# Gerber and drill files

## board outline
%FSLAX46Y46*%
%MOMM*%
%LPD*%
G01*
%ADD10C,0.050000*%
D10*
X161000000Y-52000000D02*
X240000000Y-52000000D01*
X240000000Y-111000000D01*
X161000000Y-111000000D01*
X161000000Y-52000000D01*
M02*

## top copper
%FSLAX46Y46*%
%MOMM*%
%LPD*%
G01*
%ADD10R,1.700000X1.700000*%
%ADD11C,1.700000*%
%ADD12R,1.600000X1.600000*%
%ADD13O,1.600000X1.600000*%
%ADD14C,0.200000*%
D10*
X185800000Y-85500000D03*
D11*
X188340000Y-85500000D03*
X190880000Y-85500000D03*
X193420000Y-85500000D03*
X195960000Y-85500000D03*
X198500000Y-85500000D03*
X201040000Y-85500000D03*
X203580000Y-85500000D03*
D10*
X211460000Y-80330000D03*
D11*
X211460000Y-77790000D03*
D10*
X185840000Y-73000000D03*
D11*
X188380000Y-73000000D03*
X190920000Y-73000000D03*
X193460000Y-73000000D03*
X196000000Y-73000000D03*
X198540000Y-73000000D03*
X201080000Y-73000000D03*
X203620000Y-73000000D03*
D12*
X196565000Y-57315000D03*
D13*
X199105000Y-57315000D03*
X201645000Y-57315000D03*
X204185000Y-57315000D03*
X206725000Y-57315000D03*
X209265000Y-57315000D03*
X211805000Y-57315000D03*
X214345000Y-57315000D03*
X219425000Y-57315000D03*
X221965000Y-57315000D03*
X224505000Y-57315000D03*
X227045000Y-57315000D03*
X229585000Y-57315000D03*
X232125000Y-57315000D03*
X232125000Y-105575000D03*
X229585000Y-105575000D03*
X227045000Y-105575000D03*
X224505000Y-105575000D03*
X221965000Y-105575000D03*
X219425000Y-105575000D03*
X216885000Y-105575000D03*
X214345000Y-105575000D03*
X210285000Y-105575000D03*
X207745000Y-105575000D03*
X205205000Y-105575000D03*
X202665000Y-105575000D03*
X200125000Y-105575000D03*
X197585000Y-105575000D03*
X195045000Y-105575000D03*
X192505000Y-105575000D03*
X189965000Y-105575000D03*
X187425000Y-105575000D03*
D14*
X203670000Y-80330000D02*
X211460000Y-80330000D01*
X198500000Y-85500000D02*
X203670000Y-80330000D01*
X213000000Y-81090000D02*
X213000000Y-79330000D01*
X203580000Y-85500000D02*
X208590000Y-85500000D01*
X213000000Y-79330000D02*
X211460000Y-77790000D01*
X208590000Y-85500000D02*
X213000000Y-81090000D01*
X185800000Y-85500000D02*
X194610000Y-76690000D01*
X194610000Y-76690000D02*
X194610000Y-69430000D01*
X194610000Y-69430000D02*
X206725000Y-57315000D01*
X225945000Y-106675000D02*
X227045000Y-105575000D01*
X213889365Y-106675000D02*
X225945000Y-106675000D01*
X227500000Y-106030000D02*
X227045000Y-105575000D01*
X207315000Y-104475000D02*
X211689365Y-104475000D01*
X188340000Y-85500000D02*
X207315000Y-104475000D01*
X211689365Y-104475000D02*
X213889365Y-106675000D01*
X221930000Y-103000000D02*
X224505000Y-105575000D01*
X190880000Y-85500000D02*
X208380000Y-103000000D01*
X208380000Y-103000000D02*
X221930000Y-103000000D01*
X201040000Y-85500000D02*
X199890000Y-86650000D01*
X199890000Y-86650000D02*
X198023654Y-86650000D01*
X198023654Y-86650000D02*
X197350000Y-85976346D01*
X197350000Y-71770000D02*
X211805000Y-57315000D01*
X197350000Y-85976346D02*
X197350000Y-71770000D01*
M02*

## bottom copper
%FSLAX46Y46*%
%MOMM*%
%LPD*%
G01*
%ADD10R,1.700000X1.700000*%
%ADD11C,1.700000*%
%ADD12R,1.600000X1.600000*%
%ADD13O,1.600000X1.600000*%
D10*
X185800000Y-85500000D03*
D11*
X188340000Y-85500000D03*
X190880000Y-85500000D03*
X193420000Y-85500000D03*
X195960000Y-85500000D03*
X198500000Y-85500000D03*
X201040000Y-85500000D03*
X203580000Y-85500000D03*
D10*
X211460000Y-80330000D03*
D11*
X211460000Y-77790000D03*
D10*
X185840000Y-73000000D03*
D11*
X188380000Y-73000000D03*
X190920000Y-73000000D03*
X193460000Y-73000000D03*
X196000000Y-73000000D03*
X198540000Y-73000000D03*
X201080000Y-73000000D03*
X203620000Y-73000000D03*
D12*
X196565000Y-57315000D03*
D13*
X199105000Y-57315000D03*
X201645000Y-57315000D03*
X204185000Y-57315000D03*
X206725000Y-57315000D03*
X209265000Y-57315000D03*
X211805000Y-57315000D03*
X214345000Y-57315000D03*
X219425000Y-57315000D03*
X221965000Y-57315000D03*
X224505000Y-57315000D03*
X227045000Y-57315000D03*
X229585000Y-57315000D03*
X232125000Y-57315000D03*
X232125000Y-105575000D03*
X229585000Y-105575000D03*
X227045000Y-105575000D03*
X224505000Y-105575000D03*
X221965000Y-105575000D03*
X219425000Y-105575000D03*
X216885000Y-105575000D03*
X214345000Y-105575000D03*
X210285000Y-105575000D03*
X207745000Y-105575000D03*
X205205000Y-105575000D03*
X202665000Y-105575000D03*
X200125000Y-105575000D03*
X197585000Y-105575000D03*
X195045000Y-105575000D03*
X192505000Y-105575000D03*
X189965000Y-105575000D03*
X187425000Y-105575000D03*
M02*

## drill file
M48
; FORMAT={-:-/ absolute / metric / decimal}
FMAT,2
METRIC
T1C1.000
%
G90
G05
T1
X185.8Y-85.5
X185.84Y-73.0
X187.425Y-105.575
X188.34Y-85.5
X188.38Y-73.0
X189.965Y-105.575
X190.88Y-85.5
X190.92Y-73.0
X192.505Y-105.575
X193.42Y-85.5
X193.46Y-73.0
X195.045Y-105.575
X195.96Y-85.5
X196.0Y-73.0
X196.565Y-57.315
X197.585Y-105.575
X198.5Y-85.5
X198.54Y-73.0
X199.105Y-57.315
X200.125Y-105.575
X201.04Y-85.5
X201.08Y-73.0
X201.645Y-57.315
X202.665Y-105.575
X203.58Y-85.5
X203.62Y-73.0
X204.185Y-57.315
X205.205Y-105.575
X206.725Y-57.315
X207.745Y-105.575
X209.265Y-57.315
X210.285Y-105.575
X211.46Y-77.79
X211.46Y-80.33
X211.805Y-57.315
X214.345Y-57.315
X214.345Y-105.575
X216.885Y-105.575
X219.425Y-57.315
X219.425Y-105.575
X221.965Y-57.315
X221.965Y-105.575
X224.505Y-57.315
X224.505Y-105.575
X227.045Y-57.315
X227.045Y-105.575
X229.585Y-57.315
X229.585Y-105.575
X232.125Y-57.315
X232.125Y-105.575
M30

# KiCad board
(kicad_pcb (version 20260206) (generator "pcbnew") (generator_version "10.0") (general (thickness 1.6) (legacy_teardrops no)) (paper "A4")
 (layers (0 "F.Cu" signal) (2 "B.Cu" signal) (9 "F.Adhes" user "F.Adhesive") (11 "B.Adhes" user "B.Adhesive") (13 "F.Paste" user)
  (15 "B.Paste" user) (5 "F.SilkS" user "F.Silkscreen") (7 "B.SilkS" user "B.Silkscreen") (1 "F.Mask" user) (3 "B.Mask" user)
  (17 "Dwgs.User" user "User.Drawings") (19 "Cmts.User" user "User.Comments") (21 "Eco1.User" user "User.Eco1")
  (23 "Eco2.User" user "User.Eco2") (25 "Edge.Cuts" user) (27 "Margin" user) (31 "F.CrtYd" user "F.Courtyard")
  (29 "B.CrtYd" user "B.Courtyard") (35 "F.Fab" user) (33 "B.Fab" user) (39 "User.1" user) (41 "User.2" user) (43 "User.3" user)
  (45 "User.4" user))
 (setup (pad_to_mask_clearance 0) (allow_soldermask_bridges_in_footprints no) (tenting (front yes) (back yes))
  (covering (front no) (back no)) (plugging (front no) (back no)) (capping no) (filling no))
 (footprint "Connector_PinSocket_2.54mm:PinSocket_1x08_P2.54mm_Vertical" (layer "F.Cu") (at 185.8 85.5 90)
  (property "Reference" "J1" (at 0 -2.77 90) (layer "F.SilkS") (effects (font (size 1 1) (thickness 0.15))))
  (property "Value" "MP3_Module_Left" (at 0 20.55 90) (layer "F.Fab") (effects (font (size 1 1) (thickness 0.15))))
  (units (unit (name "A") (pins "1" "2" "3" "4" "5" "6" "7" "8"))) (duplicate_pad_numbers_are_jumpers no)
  (pad "1" thru_hole rect (at 0 0 90) (size 1.7 1.7) (drill 1) (layers "*.Cu" "*.Mask") (remove_unused_layers no) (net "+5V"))
  (pad "2" thru_hole circle (at 0 2.54 90) (size 1.7 1.7) (drill 1) (layers "*.Cu" "*.Mask") (remove_unused_layers no) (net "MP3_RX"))
  (pad "3" thru_hole circle (at 0 5.08 90) (size 1.7 1.7) (drill 1) (layers "*.Cu" "*.Mask") (remove_unused_layers no) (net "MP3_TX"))
  (pad "4" thru_hole circle (at 0 7.62 90) (size 1.7 1.7) (drill 1) (layers "*.Cu" "*.Mask") (remove_unused_layers no)
   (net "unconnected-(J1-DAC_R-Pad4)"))
  (pad "5" thru_hole circle (at 0 10.16 90) (size 1.7 1.7) (drill 1) (layers "*.Cu" "*.Mask") (remove_unused_layers no)
   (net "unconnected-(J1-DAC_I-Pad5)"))
  (pad "6" thru_hole circle (at 0 12.7 90) (size 1.7 1.7) (drill 1) (layers "*.Cu" "*.Mask") (remove_unused_layers no) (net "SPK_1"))
  (pad "7" thru_hole circle (at 0 15.24 90) (size 1.7 1.7) (drill 1) (layers "*.Cu" "*.Mask") (remove_unused_layers no) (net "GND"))
  (pad "8" thru_hole circle (at 0 17.78 90) (size 1.7 1.7) (drill 1) (layers "*.Cu" "*.Mask") (remove_unused_layers no) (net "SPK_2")))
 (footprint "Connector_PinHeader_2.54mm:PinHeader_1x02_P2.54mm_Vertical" (layer "F.Cu") (at 211.46 80.33 180)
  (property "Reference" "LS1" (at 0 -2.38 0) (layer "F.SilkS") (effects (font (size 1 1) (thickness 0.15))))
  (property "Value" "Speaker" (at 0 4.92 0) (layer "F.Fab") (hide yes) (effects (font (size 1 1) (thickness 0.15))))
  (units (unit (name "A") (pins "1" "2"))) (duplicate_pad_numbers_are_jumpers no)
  (pad "1" thru_hole rect (at 0 0 180) (size 1.7 1.7) (drill 1) (layers "*.Cu" "*.Mask") (remove_unused_layers no) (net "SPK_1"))
  (pad "2" thru_hole circle (at 0 2.54 180) (size 1.7 1.7) (drill 1) (layers "*.Cu" "*.Mask") (remove_unused_layers no) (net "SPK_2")))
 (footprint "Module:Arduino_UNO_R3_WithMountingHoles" (layer "F.Cu") (at 115.75 120.70425)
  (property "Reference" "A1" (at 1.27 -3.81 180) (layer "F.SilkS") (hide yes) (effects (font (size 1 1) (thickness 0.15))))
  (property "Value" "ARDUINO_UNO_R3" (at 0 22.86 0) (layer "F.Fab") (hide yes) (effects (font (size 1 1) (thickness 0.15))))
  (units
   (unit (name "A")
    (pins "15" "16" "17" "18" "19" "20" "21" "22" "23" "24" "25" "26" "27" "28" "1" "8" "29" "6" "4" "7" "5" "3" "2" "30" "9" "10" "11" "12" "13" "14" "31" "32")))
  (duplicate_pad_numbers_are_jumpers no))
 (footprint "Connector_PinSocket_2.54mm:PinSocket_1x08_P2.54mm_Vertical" (layer "F.Cu") (at 185.84 73 90)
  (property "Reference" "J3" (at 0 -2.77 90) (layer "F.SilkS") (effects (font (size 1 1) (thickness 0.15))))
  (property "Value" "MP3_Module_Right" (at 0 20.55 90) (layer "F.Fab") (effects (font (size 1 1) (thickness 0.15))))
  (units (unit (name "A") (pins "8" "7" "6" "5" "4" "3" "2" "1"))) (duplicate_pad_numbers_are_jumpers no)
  (pad "1" thru_hole rect (at 0 0 90) (size 1.7 1.7) (drill 1) (layers "*.Cu" "*.Mask") (remove_unused_layers no)
   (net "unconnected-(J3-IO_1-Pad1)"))
  (pad "2" thru_hole circle (at 0 2.54 90) (size 1.7 1.7) (drill 1) (layers "*.Cu" "*.Mask") (remove_unused_layers no)
   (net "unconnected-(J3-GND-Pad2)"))
  (pad "3" thru_hole circle (at 0 5.08 90) (size 1.7 1.7) (drill 1) (layers "*.Cu" "*.Mask") (remove_unused_layers no)
   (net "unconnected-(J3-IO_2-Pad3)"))
  (pad "4" thru_hole circle (at 0 7.62 90) (size 1.7 1.7) (drill 1) (layers "*.Cu" "*.Mask") (remove_unused_layers no)
   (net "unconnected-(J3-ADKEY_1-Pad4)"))
  (pad "5" thru_hole circle (at 0 10.16 90) (size 1.7 1.7) (drill 1) (layers "*.Cu" "*.Mask") (remove_unused_layers no)
   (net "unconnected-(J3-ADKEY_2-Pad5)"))
  (pad "6" thru_hole circle (at 0 12.7 90) (size 1.7 1.7) (drill 1) (layers "*.Cu" "*.Mask") (remove_unused_layers no)
   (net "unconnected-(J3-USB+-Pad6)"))
  (pad "7" thru_hole circle (at 0 15.24 90) (size 1.7 1.7) (drill 1) (layers "*.Cu" "*.Mask") (remove_unused_layers no)
   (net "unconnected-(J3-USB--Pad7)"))
  (pad "8" thru_hole circle (at 0 17.78 90) (size 1.7 1.7) (drill 1) (layers "*.Cu" "*.Mask") (remove_unused_layers no)
   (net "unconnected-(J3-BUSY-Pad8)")))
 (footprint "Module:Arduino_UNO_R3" (layer "F.Cu") (at 196.565 57.315)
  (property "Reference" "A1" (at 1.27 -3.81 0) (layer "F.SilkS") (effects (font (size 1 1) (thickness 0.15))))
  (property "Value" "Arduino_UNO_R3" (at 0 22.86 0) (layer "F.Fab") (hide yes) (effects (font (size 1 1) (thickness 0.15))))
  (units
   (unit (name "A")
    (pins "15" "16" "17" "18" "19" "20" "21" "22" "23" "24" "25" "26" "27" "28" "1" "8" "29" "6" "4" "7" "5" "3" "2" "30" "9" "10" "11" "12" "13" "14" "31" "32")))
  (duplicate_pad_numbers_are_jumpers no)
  (pad "1" thru_hole rect (at 0 0 90) (size 1.6 1.6) (drill 1) (layers "*.Cu" "*.Mask") (remove_unused_layers no)
   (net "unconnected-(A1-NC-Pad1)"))
  (pad "2" thru_hole oval (at 2.54 0 90) (size 1.6 1.6) (drill 1) (layers "*.Cu" "*.Mask") (remove_unused_layers no)
   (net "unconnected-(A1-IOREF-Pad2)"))
  (pad "3" thru_hole oval (at 5.08 0 90) (size 1.6 1.6) (drill 1) (layers "*.Cu" "*.Mask") (remove_unused_layers no)
   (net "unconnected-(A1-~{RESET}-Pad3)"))
  (pad "4" thru_hole oval (at 7.62 0 90) (size 1.6 1.6) (drill 1) (layers "*.Cu" "*.Mask") (remove_unused_layers no)
   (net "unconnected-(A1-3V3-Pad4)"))
  (pad "5" thru_hole oval (at 10.16 0 90) (size 1.6 1.6) (drill 1) (layers "*.Cu" "*.Mask") (remove_unused_layers no) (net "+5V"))
  (pad "6" thru_hole oval (at 12.7 0 90) (size 1.6 1.6) (drill 1) (layers "*.Cu" "*.Mask") (remove_unused_layers no)
   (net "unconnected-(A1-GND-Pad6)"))
  (pad "7" thru_hole oval (at 15.24 0 90) (size 1.6 1.6) (drill 1) (layers "*.Cu" "*.Mask") (remove_unused_layers no) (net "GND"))
  (pad "8" thru_hole oval (at 17.78 0 90) (size 1.6 1.6) (drill 1) (layers "*.Cu" "*.Mask") (remove_unused_layers no)
   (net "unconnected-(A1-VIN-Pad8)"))
  (pad "9" thru_hole oval (at 22.86 0 90) (size 1.6 1.6) (drill 1) (layers "*.Cu" "*.Mask") (remove_unused_layers no)
   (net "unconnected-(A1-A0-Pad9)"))
  (pad "10" thru_hole oval (at 25.4 0 90) (size 1.6 1.6) (drill 1) (layers "*.Cu" "*.Mask") (remove_unused_layers no)
   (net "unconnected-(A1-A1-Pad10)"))
  (pad "11" thru_hole oval (at 27.94 0 90) (size 1.6 1.6) (drill 1) (layers "*.Cu" "*.Mask") (remove_unused_layers no)
   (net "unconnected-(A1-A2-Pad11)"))
  (pad "12" thru_hole oval (at 30.48 0 90) (size 1.6 1.6) (drill 1) (layers "*.Cu" "*.Mask") (remove_unused_layers no)
   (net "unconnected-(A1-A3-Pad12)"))
  (pad "13" thru_hole oval (at 33.02 0 90) (size 1.6 1.6) (drill 1) (layers "*.Cu" "*.Mask") (remove_unused_layers no)
   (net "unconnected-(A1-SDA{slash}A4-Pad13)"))
  (pad "14" thru_hole oval (at 35.56 0 90) (size 1.6 1.6) (drill 1) (layers "*.Cu" "*.Mask") (remove_unused_layers no)
   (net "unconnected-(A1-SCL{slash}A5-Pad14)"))
  (pad "15" thru_hole oval (at 35.56 48.26 90) (size 1.6 1.6) (drill 1) (layers "*.Cu" "*.Mask") (remove_unused_layers no)
   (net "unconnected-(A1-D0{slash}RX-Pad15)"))
  (pad "16" thru_hole oval (at 33.02 48.26 90) (size 1.6 1.6) (drill 1) (layers "*.Cu" "*.Mask") (remove_unused_layers no)
   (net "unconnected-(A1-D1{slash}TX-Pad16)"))
  (pad "17" thru_hole oval (at 30.48 48.26 90) (size 1.6 1.6) (drill 1) (layers "*.Cu" "*.Mask") (remove_unused_layers no) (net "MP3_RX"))
  (pad "18" thru_hole oval (at 27.94 48.26 90) (size 1.6 1.6) (drill 1) (layers "*.Cu" "*.Mask") (remove_unused_layers no) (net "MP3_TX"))
  (pad "19" thru_hole oval (at 25.4 48.26 90) (size 1.6 1.6) (drill 1) (layers "*.Cu" "*.Mask") (remove_unused_layers no)
   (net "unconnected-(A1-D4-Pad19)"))
  (pad "20" thru_hole oval (at 22.86 48.26 90) (size 1.6 1.6) (drill 1) (layers "*.Cu" "*.Mask") (remove_unused_layers no)
   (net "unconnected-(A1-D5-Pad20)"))
  (pad "21" thru_hole oval (at 20.32 48.26 90) (size 1.6 1.6) (drill 1) (layers "*.Cu" "*.Mask") (remove_unused_layers no)
   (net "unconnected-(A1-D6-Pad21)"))
  (pad "22" thru_hole oval (at 17.78 48.26 90) (size 1.6 1.6) (drill 1) (layers "*.Cu" "*.Mask") (remove_unused_layers no)
   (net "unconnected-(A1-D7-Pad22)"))
  (pad "23" thru_hole oval (at 13.72 48.26 90) (size 1.6 1.6) (drill 1) (layers "*.Cu" "*.Mask") (remove_unused_layers no)
   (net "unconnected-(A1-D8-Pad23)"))
  (pad "24" thru_hole oval (at 11.18 48.26 90) (size 1.6 1.6) (drill 1) (layers "*.Cu" "*.Mask") (remove_unused_layers no)
   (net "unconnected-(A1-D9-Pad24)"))
  (pad "25" thru_hole oval (at 8.64 48.26 90) (size 1.6 1.6) (drill 1) (layers "*.Cu" "*.Mask") (remove_unused_layers no)
   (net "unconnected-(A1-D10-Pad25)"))
  (pad "26" thru_hole oval (at 6.1 48.26 90) (size 1.6 1.6) (drill 1) (layers "*.Cu" "*.Mask") (remove_unused_layers no)
   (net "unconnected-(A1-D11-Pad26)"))
  (pad "27" thru_hole oval (at 3.56 48.26 90) (size 1.6 1.6) (drill 1) (layers "*.Cu" "*.Mask") (remove_unused_layers no)
   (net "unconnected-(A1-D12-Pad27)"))
  (pad "28" thru_hole oval (at 1.02 48.26 90) (size 1.6 1.6) (drill 1) (layers "*.Cu" "*.Mask") (remove_unused_layers no)
   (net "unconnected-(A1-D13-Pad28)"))
  (pad "29" thru_hole oval (at -1.52 48.26 90) (size 1.6 1.6) (drill 1) (layers "*.Cu" "*.Mask") (remove_unused_layers no)
   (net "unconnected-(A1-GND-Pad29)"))
  (pad "30" thru_hole oval (at -4.06 48.26 90) (size 1.6 1.6) (drill 1) (layers "*.Cu" "*.Mask") (remove_unused_layers no)
   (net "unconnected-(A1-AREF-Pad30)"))
  (pad "31" thru_hole oval (at -6.6 48.26 90) (size 1.6 1.6) (drill 1) (layers "*.Cu" "*.Mask") (remove_unused_layers no)
   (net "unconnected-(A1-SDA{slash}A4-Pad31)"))
  (pad "32" thru_hole oval (at -9.14 48.26 90) (size 1.6 1.6) (drill 1) (layers "*.Cu" "*.Mask") (remove_unused_layers no)
   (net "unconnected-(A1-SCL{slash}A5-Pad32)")))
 (gr_rect (start 161 52) (end 240 111) (stroke (width 0.05) (type default)) (fill no) (layer "Edge.Cuts"))
 (segment (start 203.67 80.33) (end 211.46 80.33) (width 0.2) (layer "F.Cu") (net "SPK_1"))
 (segment (start 198.5 85.5) (end 203.67 80.33) (width 0.2) (layer "F.Cu") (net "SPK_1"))
 (segment (start 213 81.09) (end 213 79.33) (width 0.2) (layer "F.Cu") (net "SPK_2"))
 (segment (start 203.58 85.5) (end 208.59 85.5) (width 0.2) (layer "F.Cu") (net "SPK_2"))
 (segment (start 213 79.33) (end 211.46 77.79) (width 0.2) (layer "F.Cu") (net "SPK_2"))
 (segment (start 208.59 85.5) (end 213 81.09) (width 0.2) (layer "F.Cu") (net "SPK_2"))
 (segment (start 185.8 85.5) (end 194.61 76.69) (width 0.2) (layer "F.Cu") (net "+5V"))
 (segment (start 194.61 76.69) (end 194.61 69.43) (width 0.2) (layer "F.Cu") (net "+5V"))
 (segment (start 194.61 69.43) (end 206.725 57.315) (width 0.2) (layer "F.Cu") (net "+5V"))
 (segment (start 225.945 106.675) (end 227.045 105.575) (width 0.2) (layer "F.Cu") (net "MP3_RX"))
 (segment (start 213.889365 106.675) (end 225.945 106.675) (width 0.2) (layer "F.Cu") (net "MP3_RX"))
 (segment (start 227.5 106.03) (end 227.045 105.575) (width 0.2) (layer "F.Cu") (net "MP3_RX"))
 (segment (start 207.315 104.475) (end 211.689365 104.475) (width 0.2) (layer "F.Cu") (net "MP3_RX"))
 (segment (start 188.34 85.5) (end 207.315 104.475) (width 0.2) (layer "F.Cu") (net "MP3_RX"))
 (segment (start 211.689365 104.475) (end 213.889365 106.675) (width 0.2) (layer "F.Cu") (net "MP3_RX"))
 (segment (start 221.93 103) (end 224.505 105.575) (width 0.2) (layer "F.Cu") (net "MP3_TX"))
 (segment (start 190.88 85.5) (end 208.38 103) (width 0.2) (layer "F.Cu") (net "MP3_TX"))
 (segment (start 208.38 103) (end 221.93 103) (width 0.2) (layer "F.Cu") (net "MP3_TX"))
 (segment (start 201.04 85.5) (end 199.89 86.65) (width 0.2) (layer "F.Cu") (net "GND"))
 (segment (start 199.89 86.65) (end 198.023654 86.65) (width 0.2) (layer "F.Cu") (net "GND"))
 (segment (start 198.023654 86.65) (end 197.35 85.976346) (width 0.2) (layer "F.Cu") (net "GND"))
 (segment (start 197.35 71.77) (end 211.805 57.315) (width 0.2) (layer "F.Cu") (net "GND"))
 (segment (start 197.35 85.976346) (end 197.35 71.77) (width 0.2) (layer "F.Cu") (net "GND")))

